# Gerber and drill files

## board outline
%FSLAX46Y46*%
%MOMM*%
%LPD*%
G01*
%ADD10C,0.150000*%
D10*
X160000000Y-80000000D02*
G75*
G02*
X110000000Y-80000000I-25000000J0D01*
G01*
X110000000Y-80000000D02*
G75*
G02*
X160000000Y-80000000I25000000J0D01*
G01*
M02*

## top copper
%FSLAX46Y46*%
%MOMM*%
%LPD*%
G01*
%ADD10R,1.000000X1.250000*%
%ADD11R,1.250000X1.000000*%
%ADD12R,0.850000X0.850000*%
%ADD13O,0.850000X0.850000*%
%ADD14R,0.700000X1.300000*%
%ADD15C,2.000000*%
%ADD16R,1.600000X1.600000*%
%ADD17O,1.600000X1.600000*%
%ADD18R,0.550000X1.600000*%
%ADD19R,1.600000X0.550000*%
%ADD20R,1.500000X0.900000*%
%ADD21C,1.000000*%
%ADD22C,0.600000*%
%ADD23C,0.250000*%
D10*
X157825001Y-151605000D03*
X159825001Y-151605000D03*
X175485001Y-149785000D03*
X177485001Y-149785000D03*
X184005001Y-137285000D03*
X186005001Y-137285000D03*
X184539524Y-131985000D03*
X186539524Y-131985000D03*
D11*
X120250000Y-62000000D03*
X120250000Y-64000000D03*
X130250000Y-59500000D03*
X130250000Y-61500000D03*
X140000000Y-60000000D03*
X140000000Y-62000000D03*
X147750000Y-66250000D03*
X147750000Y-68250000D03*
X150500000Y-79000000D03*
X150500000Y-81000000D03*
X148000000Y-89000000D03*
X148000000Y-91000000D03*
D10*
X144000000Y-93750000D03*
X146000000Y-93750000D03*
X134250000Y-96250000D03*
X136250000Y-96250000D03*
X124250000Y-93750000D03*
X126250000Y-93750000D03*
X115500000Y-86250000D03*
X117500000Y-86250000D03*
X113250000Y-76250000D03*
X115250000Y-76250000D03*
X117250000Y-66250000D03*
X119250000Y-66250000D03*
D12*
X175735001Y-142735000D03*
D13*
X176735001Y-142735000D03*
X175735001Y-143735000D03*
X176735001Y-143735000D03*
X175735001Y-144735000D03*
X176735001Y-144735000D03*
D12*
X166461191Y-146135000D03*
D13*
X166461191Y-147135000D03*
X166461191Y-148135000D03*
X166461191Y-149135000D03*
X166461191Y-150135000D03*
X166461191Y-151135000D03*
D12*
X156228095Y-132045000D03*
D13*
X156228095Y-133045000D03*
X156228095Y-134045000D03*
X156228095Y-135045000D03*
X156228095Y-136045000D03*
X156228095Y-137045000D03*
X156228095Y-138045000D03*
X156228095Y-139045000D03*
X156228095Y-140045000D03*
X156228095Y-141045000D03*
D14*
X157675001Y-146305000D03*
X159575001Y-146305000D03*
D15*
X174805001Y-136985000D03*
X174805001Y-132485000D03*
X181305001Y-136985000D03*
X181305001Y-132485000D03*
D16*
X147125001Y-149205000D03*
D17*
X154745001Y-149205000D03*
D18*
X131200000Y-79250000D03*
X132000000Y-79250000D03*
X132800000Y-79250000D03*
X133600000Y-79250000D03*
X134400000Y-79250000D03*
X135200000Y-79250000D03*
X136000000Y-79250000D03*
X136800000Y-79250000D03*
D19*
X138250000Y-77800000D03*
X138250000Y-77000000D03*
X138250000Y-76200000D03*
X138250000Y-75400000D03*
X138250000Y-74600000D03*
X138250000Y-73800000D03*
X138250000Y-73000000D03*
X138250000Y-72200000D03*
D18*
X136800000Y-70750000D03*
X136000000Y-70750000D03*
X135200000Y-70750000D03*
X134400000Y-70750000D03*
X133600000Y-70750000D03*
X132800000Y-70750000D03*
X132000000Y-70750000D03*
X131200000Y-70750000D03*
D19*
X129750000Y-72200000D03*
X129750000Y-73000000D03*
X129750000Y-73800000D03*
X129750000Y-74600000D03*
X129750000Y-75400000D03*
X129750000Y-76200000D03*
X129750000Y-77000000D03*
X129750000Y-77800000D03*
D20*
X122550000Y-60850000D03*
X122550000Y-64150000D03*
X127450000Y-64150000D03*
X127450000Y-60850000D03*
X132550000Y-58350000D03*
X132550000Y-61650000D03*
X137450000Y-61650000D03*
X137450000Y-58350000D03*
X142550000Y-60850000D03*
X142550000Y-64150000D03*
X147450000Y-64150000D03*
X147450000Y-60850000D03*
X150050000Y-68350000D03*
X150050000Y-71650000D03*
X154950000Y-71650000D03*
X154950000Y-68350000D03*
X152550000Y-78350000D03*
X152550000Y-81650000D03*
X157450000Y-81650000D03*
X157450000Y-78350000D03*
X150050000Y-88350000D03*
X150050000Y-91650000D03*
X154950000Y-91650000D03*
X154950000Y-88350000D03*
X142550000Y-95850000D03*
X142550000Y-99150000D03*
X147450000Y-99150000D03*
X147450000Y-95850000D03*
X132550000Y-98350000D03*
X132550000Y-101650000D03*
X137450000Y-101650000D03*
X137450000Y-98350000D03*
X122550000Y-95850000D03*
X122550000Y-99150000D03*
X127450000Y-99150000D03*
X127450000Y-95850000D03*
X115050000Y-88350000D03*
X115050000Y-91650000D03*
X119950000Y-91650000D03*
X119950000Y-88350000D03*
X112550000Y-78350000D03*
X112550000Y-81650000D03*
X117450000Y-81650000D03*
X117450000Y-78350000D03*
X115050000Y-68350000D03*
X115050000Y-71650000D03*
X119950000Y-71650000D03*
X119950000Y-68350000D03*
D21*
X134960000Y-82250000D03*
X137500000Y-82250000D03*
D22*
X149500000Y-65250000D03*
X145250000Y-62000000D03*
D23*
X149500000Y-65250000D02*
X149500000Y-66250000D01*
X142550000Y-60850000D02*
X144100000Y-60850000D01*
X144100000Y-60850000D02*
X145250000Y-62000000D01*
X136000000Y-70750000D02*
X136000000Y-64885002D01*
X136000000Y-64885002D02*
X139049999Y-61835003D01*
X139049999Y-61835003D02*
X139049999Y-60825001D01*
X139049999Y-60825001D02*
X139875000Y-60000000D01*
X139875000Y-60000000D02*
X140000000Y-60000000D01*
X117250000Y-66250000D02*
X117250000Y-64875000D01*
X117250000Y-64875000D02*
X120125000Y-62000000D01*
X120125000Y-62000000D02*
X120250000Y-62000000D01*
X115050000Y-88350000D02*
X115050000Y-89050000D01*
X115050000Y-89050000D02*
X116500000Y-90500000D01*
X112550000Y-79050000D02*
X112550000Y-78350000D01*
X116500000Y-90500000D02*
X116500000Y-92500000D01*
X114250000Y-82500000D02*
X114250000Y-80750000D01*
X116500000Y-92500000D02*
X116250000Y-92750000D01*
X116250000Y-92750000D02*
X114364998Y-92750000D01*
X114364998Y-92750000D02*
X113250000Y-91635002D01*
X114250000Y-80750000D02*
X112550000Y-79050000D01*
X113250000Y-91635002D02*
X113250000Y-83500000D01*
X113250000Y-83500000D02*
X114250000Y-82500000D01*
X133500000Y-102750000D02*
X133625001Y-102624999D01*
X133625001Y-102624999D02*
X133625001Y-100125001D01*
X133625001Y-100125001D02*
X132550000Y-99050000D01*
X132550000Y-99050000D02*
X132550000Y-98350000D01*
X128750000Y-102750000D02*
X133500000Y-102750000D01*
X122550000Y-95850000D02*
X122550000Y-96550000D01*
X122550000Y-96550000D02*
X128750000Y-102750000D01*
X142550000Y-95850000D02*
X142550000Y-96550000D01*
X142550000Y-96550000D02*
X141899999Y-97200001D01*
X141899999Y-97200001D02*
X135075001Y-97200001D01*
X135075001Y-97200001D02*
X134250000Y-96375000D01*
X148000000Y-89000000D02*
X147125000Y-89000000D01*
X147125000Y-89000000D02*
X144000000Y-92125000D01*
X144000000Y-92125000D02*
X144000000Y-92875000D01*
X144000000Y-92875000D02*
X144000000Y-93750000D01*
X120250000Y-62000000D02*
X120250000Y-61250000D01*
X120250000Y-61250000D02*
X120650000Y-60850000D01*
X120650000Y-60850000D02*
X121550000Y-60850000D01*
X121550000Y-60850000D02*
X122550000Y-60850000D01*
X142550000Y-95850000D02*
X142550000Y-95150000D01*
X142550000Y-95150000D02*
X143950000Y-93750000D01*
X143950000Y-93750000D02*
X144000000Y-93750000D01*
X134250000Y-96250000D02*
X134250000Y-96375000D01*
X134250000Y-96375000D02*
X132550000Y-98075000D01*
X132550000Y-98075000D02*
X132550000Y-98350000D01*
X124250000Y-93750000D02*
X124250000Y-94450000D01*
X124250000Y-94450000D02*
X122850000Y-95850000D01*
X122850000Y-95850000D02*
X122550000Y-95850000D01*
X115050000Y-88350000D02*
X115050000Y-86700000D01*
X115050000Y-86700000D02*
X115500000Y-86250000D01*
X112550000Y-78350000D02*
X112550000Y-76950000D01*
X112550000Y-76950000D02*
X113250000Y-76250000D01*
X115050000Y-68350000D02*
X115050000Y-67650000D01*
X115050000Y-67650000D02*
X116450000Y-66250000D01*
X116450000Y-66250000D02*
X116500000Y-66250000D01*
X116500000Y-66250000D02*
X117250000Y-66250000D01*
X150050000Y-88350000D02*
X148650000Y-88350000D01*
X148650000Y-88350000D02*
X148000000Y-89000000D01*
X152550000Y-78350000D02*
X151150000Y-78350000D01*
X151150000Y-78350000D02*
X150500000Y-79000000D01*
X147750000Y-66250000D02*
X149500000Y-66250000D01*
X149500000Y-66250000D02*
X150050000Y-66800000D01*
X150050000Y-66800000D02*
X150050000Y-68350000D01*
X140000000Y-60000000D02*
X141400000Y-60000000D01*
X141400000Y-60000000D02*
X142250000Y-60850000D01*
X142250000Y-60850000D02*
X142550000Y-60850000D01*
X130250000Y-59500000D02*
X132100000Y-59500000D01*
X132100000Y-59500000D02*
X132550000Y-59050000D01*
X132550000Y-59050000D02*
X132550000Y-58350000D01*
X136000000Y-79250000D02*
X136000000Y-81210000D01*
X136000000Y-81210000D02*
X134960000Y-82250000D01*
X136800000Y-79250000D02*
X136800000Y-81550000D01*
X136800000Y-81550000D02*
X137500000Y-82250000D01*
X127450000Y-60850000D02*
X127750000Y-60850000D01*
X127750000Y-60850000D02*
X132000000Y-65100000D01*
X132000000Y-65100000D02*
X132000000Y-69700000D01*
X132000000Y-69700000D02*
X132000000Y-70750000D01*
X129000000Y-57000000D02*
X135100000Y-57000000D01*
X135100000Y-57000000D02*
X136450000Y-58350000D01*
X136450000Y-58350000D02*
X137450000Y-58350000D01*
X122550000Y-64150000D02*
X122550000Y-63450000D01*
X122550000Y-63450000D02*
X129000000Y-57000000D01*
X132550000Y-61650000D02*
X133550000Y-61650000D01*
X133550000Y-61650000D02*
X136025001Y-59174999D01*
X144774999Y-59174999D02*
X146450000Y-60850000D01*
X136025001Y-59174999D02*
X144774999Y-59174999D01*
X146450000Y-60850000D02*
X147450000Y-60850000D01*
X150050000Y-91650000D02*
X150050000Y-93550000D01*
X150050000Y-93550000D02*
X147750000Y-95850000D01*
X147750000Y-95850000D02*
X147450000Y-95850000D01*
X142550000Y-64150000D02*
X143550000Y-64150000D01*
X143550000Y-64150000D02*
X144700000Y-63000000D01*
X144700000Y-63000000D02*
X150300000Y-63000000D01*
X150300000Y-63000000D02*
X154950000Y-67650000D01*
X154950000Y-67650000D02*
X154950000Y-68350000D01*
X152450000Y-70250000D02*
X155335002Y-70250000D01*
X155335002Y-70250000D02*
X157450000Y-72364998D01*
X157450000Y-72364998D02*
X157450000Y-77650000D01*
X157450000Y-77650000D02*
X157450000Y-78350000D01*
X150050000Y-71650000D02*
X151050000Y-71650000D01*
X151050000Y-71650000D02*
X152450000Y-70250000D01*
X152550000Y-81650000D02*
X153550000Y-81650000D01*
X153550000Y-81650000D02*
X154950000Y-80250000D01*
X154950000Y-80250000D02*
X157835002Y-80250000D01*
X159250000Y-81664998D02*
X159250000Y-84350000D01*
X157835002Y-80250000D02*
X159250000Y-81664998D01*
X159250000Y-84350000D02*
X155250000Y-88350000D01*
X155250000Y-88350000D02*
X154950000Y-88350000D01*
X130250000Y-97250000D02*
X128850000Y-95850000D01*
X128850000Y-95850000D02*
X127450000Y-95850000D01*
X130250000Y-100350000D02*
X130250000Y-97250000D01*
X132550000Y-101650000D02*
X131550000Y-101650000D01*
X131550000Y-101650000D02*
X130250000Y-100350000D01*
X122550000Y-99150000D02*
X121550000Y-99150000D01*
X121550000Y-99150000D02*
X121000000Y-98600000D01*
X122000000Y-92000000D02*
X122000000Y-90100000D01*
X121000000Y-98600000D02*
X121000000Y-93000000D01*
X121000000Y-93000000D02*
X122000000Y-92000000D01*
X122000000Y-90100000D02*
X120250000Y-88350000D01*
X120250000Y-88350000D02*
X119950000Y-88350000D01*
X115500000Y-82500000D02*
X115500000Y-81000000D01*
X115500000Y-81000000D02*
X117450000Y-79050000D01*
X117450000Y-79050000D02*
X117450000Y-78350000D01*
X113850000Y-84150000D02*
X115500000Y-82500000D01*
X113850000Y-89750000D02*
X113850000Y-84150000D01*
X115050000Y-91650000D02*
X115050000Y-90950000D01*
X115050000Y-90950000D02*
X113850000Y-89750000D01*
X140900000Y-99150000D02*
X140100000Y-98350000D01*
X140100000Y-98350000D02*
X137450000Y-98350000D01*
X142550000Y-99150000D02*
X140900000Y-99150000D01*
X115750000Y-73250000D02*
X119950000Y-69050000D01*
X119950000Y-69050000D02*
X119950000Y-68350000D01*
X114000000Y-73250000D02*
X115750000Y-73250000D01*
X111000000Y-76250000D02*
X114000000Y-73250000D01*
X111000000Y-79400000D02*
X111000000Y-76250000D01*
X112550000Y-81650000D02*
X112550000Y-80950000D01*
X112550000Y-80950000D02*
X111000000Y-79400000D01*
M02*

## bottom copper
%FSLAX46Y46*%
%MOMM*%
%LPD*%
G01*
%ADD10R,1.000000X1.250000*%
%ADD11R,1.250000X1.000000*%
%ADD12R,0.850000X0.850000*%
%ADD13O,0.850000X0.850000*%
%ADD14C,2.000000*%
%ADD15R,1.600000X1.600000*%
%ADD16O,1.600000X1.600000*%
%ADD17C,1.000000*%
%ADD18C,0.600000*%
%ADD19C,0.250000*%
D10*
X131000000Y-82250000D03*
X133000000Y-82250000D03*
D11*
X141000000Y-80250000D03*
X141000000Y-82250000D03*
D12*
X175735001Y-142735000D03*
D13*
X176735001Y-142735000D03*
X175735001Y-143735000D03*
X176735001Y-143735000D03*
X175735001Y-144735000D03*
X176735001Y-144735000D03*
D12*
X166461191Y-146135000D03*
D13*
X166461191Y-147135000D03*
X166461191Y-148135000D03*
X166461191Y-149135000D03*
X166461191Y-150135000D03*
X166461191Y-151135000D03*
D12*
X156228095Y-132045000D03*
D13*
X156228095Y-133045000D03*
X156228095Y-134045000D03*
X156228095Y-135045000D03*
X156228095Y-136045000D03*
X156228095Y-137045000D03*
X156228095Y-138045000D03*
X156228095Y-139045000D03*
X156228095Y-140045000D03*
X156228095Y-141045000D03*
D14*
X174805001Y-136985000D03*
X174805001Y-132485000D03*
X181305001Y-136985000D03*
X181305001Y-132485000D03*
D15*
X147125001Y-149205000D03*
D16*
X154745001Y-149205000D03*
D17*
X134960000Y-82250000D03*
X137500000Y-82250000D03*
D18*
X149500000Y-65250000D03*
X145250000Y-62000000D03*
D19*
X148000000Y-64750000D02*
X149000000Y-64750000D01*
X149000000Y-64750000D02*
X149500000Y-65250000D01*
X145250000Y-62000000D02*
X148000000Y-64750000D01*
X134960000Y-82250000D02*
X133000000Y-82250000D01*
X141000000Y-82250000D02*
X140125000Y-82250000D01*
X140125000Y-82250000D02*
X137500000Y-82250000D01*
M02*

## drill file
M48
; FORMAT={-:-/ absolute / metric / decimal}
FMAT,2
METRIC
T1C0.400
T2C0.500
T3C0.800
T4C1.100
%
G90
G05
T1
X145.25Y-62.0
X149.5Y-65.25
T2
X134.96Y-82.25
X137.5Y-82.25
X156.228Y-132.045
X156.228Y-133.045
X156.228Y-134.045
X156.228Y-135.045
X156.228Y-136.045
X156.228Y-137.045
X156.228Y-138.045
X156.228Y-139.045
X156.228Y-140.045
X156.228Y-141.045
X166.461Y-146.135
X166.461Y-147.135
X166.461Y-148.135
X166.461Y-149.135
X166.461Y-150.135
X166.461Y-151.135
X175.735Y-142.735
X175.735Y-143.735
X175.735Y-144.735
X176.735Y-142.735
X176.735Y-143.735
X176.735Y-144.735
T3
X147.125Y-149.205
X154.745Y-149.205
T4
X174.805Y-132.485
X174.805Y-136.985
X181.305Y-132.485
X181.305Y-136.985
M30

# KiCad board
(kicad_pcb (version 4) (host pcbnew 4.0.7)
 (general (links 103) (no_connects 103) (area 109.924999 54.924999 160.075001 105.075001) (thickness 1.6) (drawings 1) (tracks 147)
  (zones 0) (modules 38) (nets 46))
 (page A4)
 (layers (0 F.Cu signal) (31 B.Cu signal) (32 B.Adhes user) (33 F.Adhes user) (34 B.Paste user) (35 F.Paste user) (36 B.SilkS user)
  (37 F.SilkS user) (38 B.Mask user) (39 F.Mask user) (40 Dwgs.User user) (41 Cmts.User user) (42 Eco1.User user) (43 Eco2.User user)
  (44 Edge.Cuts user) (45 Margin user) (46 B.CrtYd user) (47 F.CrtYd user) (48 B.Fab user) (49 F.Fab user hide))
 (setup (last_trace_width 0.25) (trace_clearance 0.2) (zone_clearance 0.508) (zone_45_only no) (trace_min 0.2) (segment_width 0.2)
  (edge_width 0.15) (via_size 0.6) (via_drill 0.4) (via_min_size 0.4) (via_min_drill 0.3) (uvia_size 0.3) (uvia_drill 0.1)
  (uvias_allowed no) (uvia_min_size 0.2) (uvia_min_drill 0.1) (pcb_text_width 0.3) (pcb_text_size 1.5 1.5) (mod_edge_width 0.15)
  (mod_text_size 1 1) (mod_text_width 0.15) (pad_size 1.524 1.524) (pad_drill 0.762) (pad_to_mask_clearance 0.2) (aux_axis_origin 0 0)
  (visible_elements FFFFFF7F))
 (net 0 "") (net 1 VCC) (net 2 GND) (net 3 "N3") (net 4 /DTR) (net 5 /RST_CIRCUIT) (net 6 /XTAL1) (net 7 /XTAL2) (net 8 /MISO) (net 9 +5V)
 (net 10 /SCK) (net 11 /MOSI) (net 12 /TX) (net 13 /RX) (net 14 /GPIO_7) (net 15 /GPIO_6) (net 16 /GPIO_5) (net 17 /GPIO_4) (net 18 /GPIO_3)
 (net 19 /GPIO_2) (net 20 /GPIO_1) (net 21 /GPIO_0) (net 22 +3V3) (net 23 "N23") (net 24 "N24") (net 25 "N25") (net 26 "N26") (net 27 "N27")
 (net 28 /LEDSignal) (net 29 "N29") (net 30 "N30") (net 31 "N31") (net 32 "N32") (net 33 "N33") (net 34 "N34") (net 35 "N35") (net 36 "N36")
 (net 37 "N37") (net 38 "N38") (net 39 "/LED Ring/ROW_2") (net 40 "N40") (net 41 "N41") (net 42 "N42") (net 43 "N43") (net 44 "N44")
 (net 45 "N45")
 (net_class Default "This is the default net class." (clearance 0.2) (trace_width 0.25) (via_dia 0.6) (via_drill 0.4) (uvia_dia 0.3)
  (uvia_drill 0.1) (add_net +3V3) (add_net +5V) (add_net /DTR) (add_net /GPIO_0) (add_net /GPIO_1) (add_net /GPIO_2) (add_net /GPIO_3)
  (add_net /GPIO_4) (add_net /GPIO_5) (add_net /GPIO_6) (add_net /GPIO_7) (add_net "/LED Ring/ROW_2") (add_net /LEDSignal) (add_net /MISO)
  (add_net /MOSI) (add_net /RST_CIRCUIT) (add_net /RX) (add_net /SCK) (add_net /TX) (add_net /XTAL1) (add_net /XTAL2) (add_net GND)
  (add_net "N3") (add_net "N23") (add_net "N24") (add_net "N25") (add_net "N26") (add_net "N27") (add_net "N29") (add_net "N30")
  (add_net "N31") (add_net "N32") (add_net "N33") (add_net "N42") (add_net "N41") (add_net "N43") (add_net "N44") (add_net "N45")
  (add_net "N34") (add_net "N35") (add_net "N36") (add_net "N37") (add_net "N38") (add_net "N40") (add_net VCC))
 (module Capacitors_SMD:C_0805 (layer F.Cu) (at 158.825001 151.605)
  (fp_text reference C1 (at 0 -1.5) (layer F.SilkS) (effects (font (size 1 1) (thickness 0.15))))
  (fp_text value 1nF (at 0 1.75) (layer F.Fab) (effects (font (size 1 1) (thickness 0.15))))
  (pad 1 smd rect (at -1 0) (size 1 1.25) (layers F.Cu F.Paste F.Mask) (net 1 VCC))
  (pad 2 smd rect (at 1 0) (size 1 1.25) (layers F.Cu F.Paste F.Mask) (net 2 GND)))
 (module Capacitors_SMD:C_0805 (layer F.Cu) (at 176.485001 149.785)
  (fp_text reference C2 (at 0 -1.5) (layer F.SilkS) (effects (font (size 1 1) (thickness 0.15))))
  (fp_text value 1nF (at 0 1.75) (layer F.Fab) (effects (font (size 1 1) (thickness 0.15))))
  (pad 1 smd rect (at -1 0) (size 1 1.25) (layers F.Cu F.Paste F.Mask) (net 1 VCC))
  (pad 2 smd rect (at 1 0) (size 1 1.25) (layers F.Cu F.Paste F.Mask) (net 2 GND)))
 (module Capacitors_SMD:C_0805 (layer F.Cu) (at 185.005001 137.285)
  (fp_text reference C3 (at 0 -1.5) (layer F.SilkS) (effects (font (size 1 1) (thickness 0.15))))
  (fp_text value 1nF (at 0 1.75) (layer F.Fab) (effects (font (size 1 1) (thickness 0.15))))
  (pad 1 smd rect (at -1 0) (size 1 1.25) (layers F.Cu F.Paste F.Mask) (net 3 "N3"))
  (pad 2 smd rect (at 1 0) (size 1 1.25) (layers F.Cu F.Paste F.Mask) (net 2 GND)))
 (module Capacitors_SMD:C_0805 (layer F.Cu) (at 185.539524 131.985)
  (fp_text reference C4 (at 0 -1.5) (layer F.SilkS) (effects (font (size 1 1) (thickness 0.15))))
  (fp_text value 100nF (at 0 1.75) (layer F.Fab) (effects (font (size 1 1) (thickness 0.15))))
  (pad 1 smd rect (at -1 0) (size 1 1.25) (layers F.Cu F.Paste F.Mask) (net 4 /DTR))
  (pad 2 smd rect (at 1 0) (size 1 1.25) (layers F.Cu F.Paste F.Mask) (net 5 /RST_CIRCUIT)))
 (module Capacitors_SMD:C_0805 (layer B.Cu) (at 132 82.25)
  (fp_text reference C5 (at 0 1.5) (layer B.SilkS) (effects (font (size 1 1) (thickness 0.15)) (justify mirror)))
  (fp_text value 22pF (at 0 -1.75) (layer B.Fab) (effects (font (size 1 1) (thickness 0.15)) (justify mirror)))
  (pad 1 smd rect (at -1 0) (size 1 1.25) (layers B.Cu B.Paste B.Mask) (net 2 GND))
  (pad 2 smd rect (at 1 0) (size 1 1.25) (layers B.Cu B.Paste B.Mask) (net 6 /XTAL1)))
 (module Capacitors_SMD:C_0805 (layer B.Cu) (at 141 81.25 270)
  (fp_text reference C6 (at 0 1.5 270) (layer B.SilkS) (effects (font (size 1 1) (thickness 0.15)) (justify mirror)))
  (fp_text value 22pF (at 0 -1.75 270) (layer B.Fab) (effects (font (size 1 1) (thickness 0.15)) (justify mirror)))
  (pad 1 smd rect (at -1 0 270) (size 1 1.25) (layers B.Cu B.Paste B.Mask) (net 2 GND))
  (pad 2 smd rect (at 1 0 270) (size 1 1.25) (layers B.Cu B.Paste B.Mask) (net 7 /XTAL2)))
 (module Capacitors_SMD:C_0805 (layer F.Cu) (at 120.25 63 270)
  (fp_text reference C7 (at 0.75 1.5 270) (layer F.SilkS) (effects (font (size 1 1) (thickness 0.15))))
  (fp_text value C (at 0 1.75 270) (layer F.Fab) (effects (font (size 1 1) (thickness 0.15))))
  (pad 1 smd rect (at -1 0 270) (size 1 1.25) (layers F.Cu F.Paste F.Mask) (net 1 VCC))
  (pad 2 smd rect (at 1 0 270) (size 1 1.25) (layers F.Cu F.Paste F.Mask) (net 2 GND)))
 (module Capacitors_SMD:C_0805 (layer F.Cu) (at 130.25 60.5 270)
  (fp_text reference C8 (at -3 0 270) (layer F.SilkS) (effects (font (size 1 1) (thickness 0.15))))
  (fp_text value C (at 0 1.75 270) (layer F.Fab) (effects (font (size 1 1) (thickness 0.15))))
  (pad 1 smd rect (at -1 0 270) (size 1 1.25) (layers F.Cu F.Paste F.Mask) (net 1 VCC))
  (pad 2 smd rect (at 1 0 270) (size 1 1.25) (layers F.Cu F.Paste F.Mask) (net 2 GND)))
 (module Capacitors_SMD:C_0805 (layer F.Cu) (at 140 61 270)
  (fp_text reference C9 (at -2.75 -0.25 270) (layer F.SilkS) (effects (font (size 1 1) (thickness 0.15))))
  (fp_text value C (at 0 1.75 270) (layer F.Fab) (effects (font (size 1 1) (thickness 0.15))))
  (pad 1 smd rect (at -1 0 270) (size 1 1.25) (layers F.Cu F.Paste F.Mask) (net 1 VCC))
  (pad 2 smd rect (at 1 0 270) (size 1 1.25) (layers F.Cu F.Paste F.Mask) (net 2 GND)))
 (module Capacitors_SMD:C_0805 (layer F.Cu) (at 147.75 67.25 270)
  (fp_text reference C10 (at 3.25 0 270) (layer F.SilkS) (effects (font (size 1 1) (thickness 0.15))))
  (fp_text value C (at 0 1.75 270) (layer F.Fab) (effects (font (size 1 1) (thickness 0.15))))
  (pad 1 smd rect (at -1 0 270) (size 1 1.25) (layers F.Cu F.Paste F.Mask) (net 1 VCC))
  (pad 2 smd rect (at 1 0 270) (size 1 1.25) (layers F.Cu F.Paste F.Mask) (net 2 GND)))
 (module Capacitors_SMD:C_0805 (layer F.Cu) (at 150.5 80 270)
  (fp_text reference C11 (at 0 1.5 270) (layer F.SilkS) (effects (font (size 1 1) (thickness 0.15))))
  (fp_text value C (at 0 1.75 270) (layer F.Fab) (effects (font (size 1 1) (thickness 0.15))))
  (pad 1 smd rect (at -1 0 270) (size 1 1.25) (layers F.Cu F.Paste F.Mask) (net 1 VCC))
  (pad 2 smd rect (at 1 0 270) (size 1 1.25) (layers F.Cu F.Paste F.Mask) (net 2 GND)))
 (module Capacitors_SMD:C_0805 (layer F.Cu) (at 148 90 270)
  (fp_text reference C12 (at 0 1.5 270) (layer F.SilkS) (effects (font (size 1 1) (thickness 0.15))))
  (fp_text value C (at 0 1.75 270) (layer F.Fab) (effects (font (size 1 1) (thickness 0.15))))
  (pad 1 smd rect (at -1 0 270) (size 1 1.25) (layers F.Cu F.Paste F.Mask) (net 1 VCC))
  (pad 2 smd rect (at 1 0 270) (size 1 1.25) (layers F.Cu F.Paste F.Mask) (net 2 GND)))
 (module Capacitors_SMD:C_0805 (layer F.Cu) (at 145 93.75)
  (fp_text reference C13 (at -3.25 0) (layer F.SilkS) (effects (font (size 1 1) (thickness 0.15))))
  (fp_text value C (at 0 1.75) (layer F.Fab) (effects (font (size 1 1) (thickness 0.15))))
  (pad 1 smd rect (at -1 0) (size 1 1.25) (layers F.Cu F.Paste F.Mask) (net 1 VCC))
  (pad 2 smd rect (at 1 0) (size 1 1.25) (layers F.Cu F.Paste F.Mask) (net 2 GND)))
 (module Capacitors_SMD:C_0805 (layer F.Cu) (at 135.25 96.25)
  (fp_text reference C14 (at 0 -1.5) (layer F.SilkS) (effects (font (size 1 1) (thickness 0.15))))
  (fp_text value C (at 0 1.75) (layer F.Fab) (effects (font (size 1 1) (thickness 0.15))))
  (pad 1 smd rect (at -1 0) (size 1 1.25) (layers F.Cu F.Paste F.Mask) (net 1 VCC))
  (pad 2 smd rect (at 1 0) (size 1 1.25) (layers F.Cu F.Paste F.Mask) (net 2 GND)))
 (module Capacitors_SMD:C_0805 (layer F.Cu) (at 125.25 93.75)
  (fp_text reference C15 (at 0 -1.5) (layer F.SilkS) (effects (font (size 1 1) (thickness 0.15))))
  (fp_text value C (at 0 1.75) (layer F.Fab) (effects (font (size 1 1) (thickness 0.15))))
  (pad 1 smd rect (at -1 0) (size 1 1.25) (layers F.Cu F.Paste F.Mask) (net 1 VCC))
  (pad 2 smd rect (at 1 0) (size 1 1.25) (layers F.Cu F.Paste F.Mask) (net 2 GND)))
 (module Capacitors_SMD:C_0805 (layer F.Cu) (at 116.5 86.25)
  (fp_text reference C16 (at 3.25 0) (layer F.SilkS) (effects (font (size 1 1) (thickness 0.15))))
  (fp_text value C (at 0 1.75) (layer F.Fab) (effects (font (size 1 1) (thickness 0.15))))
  (pad 1 smd rect (at -1 0) (size 1 1.25) (layers F.Cu F.Paste F.Mask) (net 1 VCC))
  (pad 2 smd rect (at 1 0) (size 1 1.25) (layers F.Cu F.Paste F.Mask) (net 2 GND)))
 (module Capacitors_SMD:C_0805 (layer F.Cu) (at 114.25 76.25)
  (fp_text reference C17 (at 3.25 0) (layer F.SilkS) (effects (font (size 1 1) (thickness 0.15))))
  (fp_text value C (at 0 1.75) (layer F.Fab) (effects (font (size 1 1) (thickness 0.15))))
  (pad 1 smd rect (at -1 0) (size 1 1.25) (layers F.Cu F.Paste F.Mask) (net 1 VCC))
  (pad 2 smd rect (at 1 0) (size 1 1.25) (layers F.Cu F.Paste F.Mask) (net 2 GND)))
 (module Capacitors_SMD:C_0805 (layer F.Cu) (at 118.25 66.25)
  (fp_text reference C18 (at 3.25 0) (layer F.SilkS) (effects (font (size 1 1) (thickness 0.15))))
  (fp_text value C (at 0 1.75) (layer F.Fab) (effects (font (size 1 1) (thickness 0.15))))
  (pad 1 smd rect (at -1 0) (size 1 1.25) (layers F.Cu F.Paste F.Mask) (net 1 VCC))
  (pad 2 smd rect (at 1 0) (size 1 1.25) (layers F.Cu F.Paste F.Mask) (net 2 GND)))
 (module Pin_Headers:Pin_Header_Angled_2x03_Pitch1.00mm (layer F.Cu) (at 175.735001 142.735)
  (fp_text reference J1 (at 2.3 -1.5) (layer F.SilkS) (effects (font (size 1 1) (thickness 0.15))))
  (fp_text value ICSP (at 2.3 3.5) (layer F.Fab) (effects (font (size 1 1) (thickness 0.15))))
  (pad 1 thru_hole rect (at 0 0) (size 0.85 0.85) (drill 0.5) (layers *.Cu *.Mask) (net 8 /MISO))
  (pad 2 thru_hole oval (at 1 0) (size 0.85 0.85) (drill 0.5) (layers *.Cu *.Mask) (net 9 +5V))
  (pad 3 thru_hole oval (at 0 1) (size 0.85 0.85) (drill 0.5) (layers *.Cu *.Mask) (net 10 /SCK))
  (pad 4 thru_hole oval (at 1 1) (size 0.85 0.85) (drill 0.5) (layers *.Cu *.Mask) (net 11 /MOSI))
  (pad 5 thru_hole oval (at 0 2) (size 0.85 0.85) (drill 0.5) (layers *.Cu *.Mask) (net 5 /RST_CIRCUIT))
  (pad 6 thru_hole oval (at 1 2) (size 0.85 0.85) (drill 0.5) (layers *.Cu *.Mask) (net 2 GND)))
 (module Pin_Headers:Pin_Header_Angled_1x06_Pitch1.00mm (layer F.Cu) (at 166.461191 146.135)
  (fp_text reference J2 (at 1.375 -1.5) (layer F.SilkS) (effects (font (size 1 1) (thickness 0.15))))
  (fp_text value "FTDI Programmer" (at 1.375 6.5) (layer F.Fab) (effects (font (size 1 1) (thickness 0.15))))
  (pad 1 thru_hole rect (at 0 0) (size 0.85 0.85) (drill 0.5) (layers *.Cu *.Mask) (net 4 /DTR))
  (pad 2 thru_hole oval (at 0 1) (size 0.85 0.85) (drill 0.5) (layers *.Cu *.Mask) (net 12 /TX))
  (pad 3 thru_hole oval (at 0 2) (size 0.85 0.85) (drill 0.5) (layers *.Cu *.Mask) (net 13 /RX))
  (pad 4 thru_hole oval (at 0 3) (size 0.85 0.85) (drill 0.5) (layers *.Cu *.Mask) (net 9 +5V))
  (pad 5 thru_hole oval (at 0 4) (size 0.85 0.85) (drill 0.5) (layers *.Cu *.Mask) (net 2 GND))
  (pad 6 thru_hole oval (at 0 5) (size 0.85 0.85) (drill 0.5) (layers *.Cu *.Mask) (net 2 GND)))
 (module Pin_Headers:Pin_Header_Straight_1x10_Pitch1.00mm (layer F.Cu) (at 156.228095 132.045)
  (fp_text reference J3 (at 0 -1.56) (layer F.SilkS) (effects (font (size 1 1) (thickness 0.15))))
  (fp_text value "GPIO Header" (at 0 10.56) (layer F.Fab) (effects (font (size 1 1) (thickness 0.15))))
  (pad 1 thru_hole rect (at 0 0) (size 0.85 0.85) (drill 0.5) (layers *.Cu *.Mask) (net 2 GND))
  (pad 2 thru_hole oval (at 0 1) (size 0.85 0.85) (drill 0.5) (layers *.Cu *.Mask) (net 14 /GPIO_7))
  (pad 3 thru_hole oval (at 0 2) (size 0.85 0.85) (drill 0.5) (layers *.Cu *.Mask) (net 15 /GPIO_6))
  (pad 4 thru_hole oval (at 0 3) (size 0.85 0.85) (drill 0.5) (layers *.Cu *.Mask) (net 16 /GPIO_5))
  (pad 5 thru_hole oval (at 0 4) (size 0.85 0.85) (drill 0.5) (layers *.Cu *.Mask) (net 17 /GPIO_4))
  (pad 6 thru_hole oval (at 0 5) (size 0.85 0.85) (drill 0.5) (layers *.Cu *.Mask) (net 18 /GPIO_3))
  (pad 7 thru_hole oval (at 0 6) (size 0.85 0.85) (drill 0.5) (layers *.Cu *.Mask) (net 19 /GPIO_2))
  (pad 8 thru_hole oval (at 0 7) (size 0.85 0.85) (drill 0.5) (layers *.Cu *.Mask) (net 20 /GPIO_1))
  (pad 9 thru_hole oval (at 0 8) (size 0.85 0.85) (drill 0.5) (layers *.Cu *.Mask) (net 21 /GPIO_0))
  (pad 10 thru_hole oval (at 0 9) (size 0.85 0.85) (drill 0.5) (layers *.Cu *.Mask) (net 1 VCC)))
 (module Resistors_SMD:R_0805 (layer F.Cu) (at 158.625001 146.305)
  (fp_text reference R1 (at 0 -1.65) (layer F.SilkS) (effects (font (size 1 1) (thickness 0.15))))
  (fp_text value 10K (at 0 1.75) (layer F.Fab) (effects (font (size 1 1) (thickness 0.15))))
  (pad 1 smd rect (at -0.95 0) (size 0.7 1.3) (layers F.Cu F.Paste F.Mask) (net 9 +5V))
  (pad 2 smd rect (at 0.95 0) (size 0.7 1.3) (layers F.Cu F.Paste F.Mask) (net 5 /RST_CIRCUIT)))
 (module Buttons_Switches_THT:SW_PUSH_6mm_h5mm (layer F.Cu) (at 174.805001 132.485)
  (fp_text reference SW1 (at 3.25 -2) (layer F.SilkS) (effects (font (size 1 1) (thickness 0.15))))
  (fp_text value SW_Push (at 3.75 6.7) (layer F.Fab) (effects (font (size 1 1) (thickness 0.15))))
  (pad 2 thru_hole circle (at 0 4.5 90) (size 2 2) (drill 1.1) (layers *.Cu *.Mask) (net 2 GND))
  (pad 1 thru_hole circle (at 0 0 90) (size 2 2) (drill 1.1) (layers *.Cu *.Mask) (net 5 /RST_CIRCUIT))
  (pad 2 thru_hole circle (at 6.5 4.5 90) (size 2 2) (drill 1.1) (layers *.Cu *.Mask) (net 2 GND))
  (pad 1 thru_hole circle (at 6.5 0 90) (size 2 2) (drill 1.1) (layers *.Cu *.Mask) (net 5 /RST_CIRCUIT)))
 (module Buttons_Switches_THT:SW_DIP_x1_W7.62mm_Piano (layer F.Cu) (at 147.125001 149.205)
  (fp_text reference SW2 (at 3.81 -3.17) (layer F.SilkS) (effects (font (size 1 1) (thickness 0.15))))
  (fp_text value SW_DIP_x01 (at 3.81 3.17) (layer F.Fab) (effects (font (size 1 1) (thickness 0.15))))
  (pad 1 thru_hole rect (at 0 0) (size 1.6 1.6) (drill 0.8) (layers *.Cu *.Mask) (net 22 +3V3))
  (pad 2 thru_hole oval (at 7.62 0) (size 1.6 1.6) (drill 0.8) (layers *.Cu *.Mask) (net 1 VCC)))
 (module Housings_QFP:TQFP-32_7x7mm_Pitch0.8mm (layer F.Cu) (at 134 75 90)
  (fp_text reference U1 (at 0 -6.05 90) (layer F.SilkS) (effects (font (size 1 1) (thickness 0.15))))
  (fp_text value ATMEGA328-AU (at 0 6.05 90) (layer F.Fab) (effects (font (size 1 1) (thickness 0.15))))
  (pad 1 smd rect (at -4.25 -2.8 90) (size 1.6 0.55) (layers F.Cu F.Paste F.Mask) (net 18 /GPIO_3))
  (pad 2 smd rect (at -4.25 -2 90) (size 1.6 0.55) (layers F.Cu F.Paste F.Mask) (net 17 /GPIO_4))
  (pad 3 smd rect (at -4.25 -1.2 90) (size 1.6 0.55) (layers F.Cu F.Paste F.Mask) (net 2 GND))
  (pad 4 smd rect (at -4.25 -0.4 90) (size 1.6 0.55) (layers F.Cu F.Paste F.Mask) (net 1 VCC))
  (pad 5 smd rect (at -4.25 0.4 90) (size 1.6 0.55) (layers F.Cu F.Paste F.Mask) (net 2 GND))
  (pad 6 smd rect (at -4.25 1.2 90) (size 1.6 0.55) (layers F.Cu F.Paste F.Mask) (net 1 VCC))
  (pad 7 smd rect (at -4.25 2 90) (size 1.6 0.55) (layers F.Cu F.Paste F.Mask) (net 6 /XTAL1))
  (pad 8 smd rect (at -4.25 2.8 90) (size 1.6 0.55) (layers F.Cu F.Paste F.Mask) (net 7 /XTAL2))
  (pad 9 smd rect (at -2.8 4.25 180) (size 1.6 0.55) (layers F.Cu F.Paste F.Mask) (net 16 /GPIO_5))
  (pad 10 smd rect (at -2 4.25 180) (size 1.6 0.55) (layers F.Cu F.Paste F.Mask) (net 15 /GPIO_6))
  (pad 11 smd rect (at -1.2 4.25 180) (size 1.6 0.55) (layers F.Cu F.Paste F.Mask) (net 14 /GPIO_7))
  (pad 12 smd rect (at -0.4 4.25 180) (size 1.6 0.55) (layers F.Cu F.Paste F.Mask) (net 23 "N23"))
  (pad 13 smd rect (at 0.4 4.25 180) (size 1.6 0.55) (layers F.Cu F.Paste F.Mask) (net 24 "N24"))
  (pad 14 smd rect (at 1.2 4.25 180) (size 1.6 0.55) (layers F.Cu F.Paste F.Mask) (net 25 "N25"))
  (pad 15 smd rect (at 2 4.25 180) (size 1.6 0.55) (layers F.Cu F.Paste F.Mask) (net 11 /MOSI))
  (pad 16 smd rect (at 2.8 4.25 180) (size 1.6 0.55) (layers F.Cu F.Paste F.Mask) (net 8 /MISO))
  (pad 17 smd rect (at 4.25 2.8 90) (size 1.6 0.55) (layers F.Cu F.Paste F.Mask) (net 10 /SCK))
  (pad 18 smd rect (at 4.25 2 90) (size 1.6 0.55) (layers F.Cu F.Paste F.Mask) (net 1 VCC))
  (pad 19 smd rect (at 4.25 1.2 90) (size 1.6 0.55) (layers F.Cu F.Paste F.Mask) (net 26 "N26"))
  (pad 20 smd rect (at 4.25 0.4 90) (size 1.6 0.55) (layers F.Cu F.Paste F.Mask) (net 3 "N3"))
  (pad 21 smd rect (at 4.25 -0.4 90) (size 1.6 0.55) (layers F.Cu F.Paste F.Mask) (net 2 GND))
  (pad 22 smd rect (at 4.25 -1.2 90) (size 1.6 0.55) (layers F.Cu F.Paste F.Mask) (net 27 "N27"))
  (pad 23 smd rect (at 4.25 -2 90) (size 1.6 0.55) (layers F.Cu F.Paste F.Mask) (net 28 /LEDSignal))
  (pad 24 smd rect (at 4.25 -2.8 90) (size 1.6 0.55) (layers F.Cu F.Paste F.Mask) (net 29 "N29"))
  (pad 25 smd rect (at 2.8 -4.25 180) (size 1.6 0.55) (layers F.Cu F.Paste F.Mask) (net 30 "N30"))
  (pad 26 smd rect (at 2 -4.25 180) (size 1.6 0.55) (layers F.Cu F.Paste F.Mask) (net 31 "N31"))
  (pad 27 smd rect (at 1.2 -4.25 180) (size 1.6 0.55) (layers F.Cu F.Paste F.Mask) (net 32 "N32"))
  (pad 28 smd rect (at 0.4 -4.25 180) (size 1.6 0.55) (layers F.Cu F.Paste F.Mask) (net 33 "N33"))
  (pad 29 smd rect (at -0.4 -4.25 180) (size 1.6 0.55) (layers F.Cu F.Paste F.Mask) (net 5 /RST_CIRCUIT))
  (pad 30 smd rect (at -1.2 -4.25 180) (size 1.6 0.55) (layers F.Cu F.Paste F.Mask) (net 21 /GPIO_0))
  (pad 31 smd rect (at -2 -4.25 180) (size 1.6 0.55) (layers F.Cu F.Paste F.Mask) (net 20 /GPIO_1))
  (pad 32 smd rect (at -2.8 -4.25 180) (size 1.6 0.55) (layers F.Cu F.Paste F.Mask) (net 19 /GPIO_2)))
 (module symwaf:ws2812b (layer F.Cu) (at 125 62.5)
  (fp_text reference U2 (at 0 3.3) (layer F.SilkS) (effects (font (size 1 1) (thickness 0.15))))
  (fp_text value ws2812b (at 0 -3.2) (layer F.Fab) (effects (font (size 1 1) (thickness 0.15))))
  (pad 1 smd rect (at -2.45 -1.65) (size 1.5 0.9) (layers F.Cu F.Paste F.Mask) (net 1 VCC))
  (pad 2 smd rect (at -2.45 1.65) (size 1.5 0.9) (layers F.Cu F.Paste F.Mask) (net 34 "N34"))
  (pad 3 smd rect (at 2.45 1.65) (size 1.5 0.9) (layers F.Cu F.Paste F.Mask) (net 2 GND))
  (pad 4 smd rect (at 2.45 -1.65) (size 1.5 0.9) (layers F.Cu F.Paste F.Mask) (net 28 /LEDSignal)))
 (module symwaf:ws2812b (layer F.Cu) (at 135 60)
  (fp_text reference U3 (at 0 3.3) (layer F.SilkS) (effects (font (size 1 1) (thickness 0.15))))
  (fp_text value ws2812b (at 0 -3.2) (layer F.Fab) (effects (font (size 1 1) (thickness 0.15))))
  (pad 1 smd rect (at -2.45 -1.65) (size 1.5 0.9) (layers F.Cu F.Paste F.Mask) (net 1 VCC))
  (pad 2 smd rect (at -2.45 1.65) (size 1.5 0.9) (layers F.Cu F.Paste F.Mask) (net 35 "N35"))
  (pad 3 smd rect (at 2.45 1.65) (size 1.5 0.9) (layers F.Cu F.Paste F.Mask) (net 2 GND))
  (pad 4 smd rect (at 2.45 -1.65) (size 1.5 0.9) (layers F.Cu F.Paste F.Mask) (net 34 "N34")))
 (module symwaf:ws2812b (layer F.Cu) (at 145 62.5)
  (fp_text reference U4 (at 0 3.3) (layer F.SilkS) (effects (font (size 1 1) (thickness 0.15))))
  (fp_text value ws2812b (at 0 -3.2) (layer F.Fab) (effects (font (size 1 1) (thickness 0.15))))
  (pad 1 smd rect (at -2.45 -1.65) (size 1.5 0.9) (layers F.Cu F.Paste F.Mask) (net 1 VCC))
  (pad 2 smd rect (at -2.45 1.65) (size 1.5 0.9) (layers F.Cu F.Paste F.Mask) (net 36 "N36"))
  (pad 3 smd rect (at 2.45 1.65) (size 1.5 0.9) (layers F.Cu F.Paste F.Mask) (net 2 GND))
  (pad 4 smd rect (at 2.45 -1.65) (size 1.5 0.9) (layers F.Cu F.Paste F.Mask) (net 35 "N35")))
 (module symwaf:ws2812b (layer F.Cu) (at 152.5 70)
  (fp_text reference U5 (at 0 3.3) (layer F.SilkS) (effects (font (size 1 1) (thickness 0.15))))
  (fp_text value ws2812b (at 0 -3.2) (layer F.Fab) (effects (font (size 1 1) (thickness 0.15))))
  (pad 1 smd rect (at -2.45 -1.65) (size 1.5 0.9) (layers F.Cu F.Paste F.Mask) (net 1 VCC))
  (pad 2 smd rect (at -2.45 1.65) (size 1.5 0.9) (layers F.Cu F.Paste F.Mask) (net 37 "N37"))
  (pad 3 smd rect (at 2.45 1.65) (size 1.5 0.9) (layers F.Cu F.Paste F.Mask) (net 2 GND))
  (pad 4 smd rect (at 2.45 -1.65) (size 1.5 0.9) (layers F.Cu F.Paste F.Mask) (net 36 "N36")))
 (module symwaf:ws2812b (layer F.Cu) (at 155 80)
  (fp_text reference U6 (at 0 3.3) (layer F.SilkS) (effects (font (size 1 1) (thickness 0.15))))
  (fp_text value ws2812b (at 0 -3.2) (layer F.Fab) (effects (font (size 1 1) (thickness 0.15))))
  (pad 1 smd rect (at -2.45 -1.65) (size 1.5 0.9) (layers F.Cu F.Paste F.Mask) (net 1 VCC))
  (pad 2 smd rect (at -2.45 1.65) (size 1.5 0.9) (layers F.Cu F.Paste F.Mask) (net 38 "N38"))
  (pad 3 smd rect (at 2.45 1.65) (size 1.5 0.9) (layers F.Cu F.Paste F.Mask) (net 2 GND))
  (pad 4 smd rect (at 2.45 -1.65) (size 1.5 0.9) (layers F.Cu F.Paste F.Mask) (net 37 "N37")))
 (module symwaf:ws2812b (layer F.Cu) (at 152.5 90)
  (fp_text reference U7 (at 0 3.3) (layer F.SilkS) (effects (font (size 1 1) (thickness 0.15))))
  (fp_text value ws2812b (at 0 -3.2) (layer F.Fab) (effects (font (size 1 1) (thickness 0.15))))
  (pad 1 smd rect (at -2.45 -1.65) (size 1.5 0.9) (layers F.Cu F.Paste F.Mask) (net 1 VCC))
  (pad 2 smd rect (at -2.45 1.65) (size 1.5 0.9) (layers F.Cu F.Paste F.Mask) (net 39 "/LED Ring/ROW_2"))
  (pad 3 smd rect (at 2.45 1.65) (size 1.5 0.9) (layers F.Cu F.Paste F.Mask) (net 2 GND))
  (pad 4 smd rect (at 2.45 -1.65) (size 1.5 0.9) (layers F.Cu F.Paste F.Mask) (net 38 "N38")))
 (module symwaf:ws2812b (layer F.Cu) (at 145 97.5)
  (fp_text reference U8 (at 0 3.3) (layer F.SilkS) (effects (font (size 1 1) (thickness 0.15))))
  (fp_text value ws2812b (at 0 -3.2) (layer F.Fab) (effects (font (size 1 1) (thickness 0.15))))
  (pad 1 smd rect (at -2.45 -1.65) (size 1.5 0.9) (layers F.Cu F.Paste F.Mask) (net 1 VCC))
  (pad 2 smd rect (at -2.45 1.65) (size 1.5 0.9) (layers F.Cu F.Paste F.Mask) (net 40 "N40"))
  (pad 3 smd rect (at 2.45 1.65) (size 1.5 0.9) (layers F.Cu F.Paste F.Mask) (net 2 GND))
  (pad 4 smd rect (at 2.45 -1.65) (size 1.5 0.9) (layers F.Cu F.Paste F.Mask) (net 39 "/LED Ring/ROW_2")))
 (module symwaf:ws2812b (layer F.Cu) (at 135 100)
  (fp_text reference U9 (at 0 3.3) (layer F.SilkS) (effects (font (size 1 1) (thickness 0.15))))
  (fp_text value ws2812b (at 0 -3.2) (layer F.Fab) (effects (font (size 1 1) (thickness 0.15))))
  (pad 1 smd rect (at -2.45 -1.65) (size 1.5 0.9) (layers F.Cu F.Paste F.Mask) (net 1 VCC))
  (pad 2 smd rect (at -2.45 1.65) (size 1.5 0.9) (layers F.Cu F.Paste F.Mask) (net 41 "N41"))
  (pad 3 smd rect (at 2.45 1.65) (size 1.5 0.9) (layers F.Cu F.Paste F.Mask) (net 2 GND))
  (pad 4 smd rect (at 2.45 -1.65) (size 1.5 0.9) (layers F.Cu F.Paste F.Mask) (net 40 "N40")))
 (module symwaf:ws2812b (layer F.Cu) (at 125 97.5)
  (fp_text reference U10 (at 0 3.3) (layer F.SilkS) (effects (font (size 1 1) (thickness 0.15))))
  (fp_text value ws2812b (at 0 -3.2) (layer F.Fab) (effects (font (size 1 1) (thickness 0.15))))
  (pad 1 smd rect (at -2.45 -1.65) (size 1.5 0.9) (layers F.Cu F.Paste F.Mask) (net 1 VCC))
  (pad 2 smd rect (at -2.45 1.65) (size 1.5 0.9) (layers F.Cu F.Paste F.Mask) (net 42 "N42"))
  (pad 3 smd rect (at 2.45 1.65) (size 1.5 0.9) (layers F.Cu F.Paste F.Mask) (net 2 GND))
  (pad 4 smd rect (at 2.45 -1.65) (size 1.5 0.9) (layers F.Cu F.Paste F.Mask) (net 41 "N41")))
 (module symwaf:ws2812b (layer F.Cu) (at 117.5 90)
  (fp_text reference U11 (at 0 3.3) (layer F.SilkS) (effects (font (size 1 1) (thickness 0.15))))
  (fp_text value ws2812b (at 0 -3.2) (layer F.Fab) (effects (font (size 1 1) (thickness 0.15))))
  (pad 1 smd rect (at -2.45 -1.65) (size 1.5 0.9) (layers F.Cu F.Paste F.Mask) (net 1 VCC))
  (pad 2 smd rect (at -2.45 1.65) (size 1.5 0.9) (layers F.Cu F.Paste F.Mask) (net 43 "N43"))
  (pad 3 smd rect (at 2.45 1.65) (size 1.5 0.9) (layers F.Cu F.Paste F.Mask) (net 2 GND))
  (pad 4 smd rect (at 2.45 -1.65) (size 1.5 0.9) (layers F.Cu F.Paste F.Mask) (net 42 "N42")))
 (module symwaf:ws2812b (layer F.Cu) (at 115 80)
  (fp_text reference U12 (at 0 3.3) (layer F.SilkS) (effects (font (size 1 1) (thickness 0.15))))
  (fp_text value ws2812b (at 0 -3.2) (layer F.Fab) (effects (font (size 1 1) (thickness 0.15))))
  (pad 1 smd rect (at -2.45 -1.65) (size 1.5 0.9) (layers F.Cu F.Paste F.Mask) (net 1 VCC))
  (pad 2 smd rect (at -2.45 1.65) (size 1.5 0.9) (layers F.Cu F.Paste F.Mask) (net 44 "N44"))
  (pad 3 smd rect (at 2.45 1.65) (size 1.5 0.9) (layers F.Cu F.Paste F.Mask) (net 2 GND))
  (pad 4 smd rect (at 2.45 -1.65) (size 1.5 0.9) (layers F.Cu F.Paste F.Mask) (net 43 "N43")))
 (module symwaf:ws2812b (layer F.Cu) (at 117.5 70)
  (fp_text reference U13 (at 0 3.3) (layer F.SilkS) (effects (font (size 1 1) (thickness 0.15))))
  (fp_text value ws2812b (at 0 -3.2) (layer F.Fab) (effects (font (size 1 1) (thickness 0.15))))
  (pad 1 smd rect (at -2.45 -1.65) (size 1.5 0.9) (layers F.Cu F.Paste F.Mask) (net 1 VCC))
  (pad 2 smd rect (at -2.45 1.65) (size 1.5 0.9) (layers F.Cu F.Paste F.Mask) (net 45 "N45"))
  (pad 3 smd rect (at 2.45 1.65) (size 1.5 0.9) (layers F.Cu F.Paste F.Mask) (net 2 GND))
  (pad 4 smd rect (at 2.45 -1.65) (size 1.5 0.9) (layers F.Cu F.Paste F.Mask) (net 44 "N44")))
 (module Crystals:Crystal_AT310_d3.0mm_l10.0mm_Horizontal (layer B.Cu) (at 134.96 82.25)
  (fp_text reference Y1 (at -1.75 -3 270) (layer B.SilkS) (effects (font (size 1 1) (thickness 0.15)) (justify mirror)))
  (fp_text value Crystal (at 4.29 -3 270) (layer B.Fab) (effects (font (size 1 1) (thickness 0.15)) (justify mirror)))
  (pad 1 thru_hole circle (at 0 0) (size 1 1) (drill 0.5) (layers *.Cu *.Mask) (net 6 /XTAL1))
  (pad 2 thru_hole circle (at 2.54 0) (size 1 1) (drill 0.5) (layers *.Cu *.Mask) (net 7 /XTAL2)))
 (gr_circle (center 135 80) (end 160 80) (layer Edge.Cuts) (width 0.15))
 (segment (start 149.5 65.25) (end 149.5 66.25) (width 0.25) (layer F.Cu) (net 1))
 (segment (start 148 64.75) (end 149 64.75) (width 0.25) (layer B.Cu) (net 1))
 (segment (start 149 64.75) (end 149.5 65.25) (width 0.25) (layer B.Cu) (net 1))
 (via (at 149.5 65.25) (size 0.6) (drill 0.4) (layers F.Cu B.Cu) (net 1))
 (segment (start 145.25 62) (end 148 64.75) (width 0.25) (layer B.Cu) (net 1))
 (segment (start 142.55 60.85) (end 144.1 60.85) (width 0.25) (layer F.Cu) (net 1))
 (segment (start 144.1 60.85) (end 145.25 62) (width 0.25) (layer F.Cu) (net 1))
 (via (at 145.25 62) (size 0.6) (drill 0.4) (layers F.Cu B.Cu) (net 1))
 (segment (start 136 70.75) (end 136 64.885002) (width 0.25) (layer F.Cu) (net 1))
 (segment (start 136 64.885002) (end 139.049999 61.835003) (width 0.25) (layer F.Cu) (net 1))
 (segment (start 139.049999 61.835003) (end 139.049999 60.825001) (width 0.25) (layer F.Cu) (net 1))
 (segment (start 139.049999 60.825001) (end 139.875 60) (width 0.25) (layer F.Cu) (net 1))
 (segment (start 139.875 60) (end 140 60) (width 0.25) (layer F.Cu) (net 1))
 (segment (start 117.25 66.25) (end 117.25 64.875) (width 0.25) (layer F.Cu) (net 1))
 (segment (start 117.25 64.875) (end 120.125 62) (width 0.25) (layer F.Cu) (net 1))
 (segment (start 120.125 62) (end 120.25 62) (width 0.25) (layer F.Cu) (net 1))
 (segment (start 115.05 88.35) (end 115.05 89.05) (width 0.25) (layer F.Cu) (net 1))
 (segment (start 115.05 89.05) (end 116.5 90.5) (width 0.25) (layer F.Cu) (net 1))
 (segment (start 112.55 79.05) (end 112.55 78.35) (width 0.25) (layer F.Cu) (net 1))
 (segment (start 116.5 90.5) (end 116.5 92.5) (width 0.25) (layer F.Cu) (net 1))
 (segment (start 114.25 82.5) (end 114.25 80.75) (width 0.25) (layer F.Cu) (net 1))
 (segment (start 116.5 92.5) (end 116.25 92.75) (width 0.25) (layer F.Cu) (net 1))
 (segment (start 116.25 92.75) (end 114.364998 92.75) (width 0.25) (layer F.Cu) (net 1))
 (segment (start 114.364998 92.75) (end 113.25 91.635002) (width 0.25) (layer F.Cu) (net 1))
 (segment (start 114.25 80.75) (end 112.55 79.05) (width 0.25) (layer F.Cu) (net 1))
 (segment (start 113.25 91.635002) (end 113.25 83.5) (width 0.25) (layer F.Cu) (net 1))
 (segment (start 113.25 83.5) (end 114.25 82.5) (width 0.25) (layer F.Cu) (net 1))
 (segment (start 133.5 102.75) (end 133.625001 102.624999) (width 0.25) (layer F.Cu) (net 1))
 (segment (start 133.625001 102.624999) (end 133.625001 100.125001) (width 0.25) (layer F.Cu) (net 1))
 (segment (start 133.625001 100.125001) (end 132.55 99.05) (width 0.25) (layer F.Cu) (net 1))
 (segment (start 132.55 99.05) (end 132.55 98.35) (width 0.25) (layer F.Cu) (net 1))
 (segment (start 128.75 102.75) (end 133.5 102.75) (width 0.25) (layer F.Cu) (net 1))
 (segment (start 122.55 95.85) (end 122.55 96.55) (width 0.25) (layer F.Cu) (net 1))
 (segment (start 122.55 96.55) (end 128.75 102.75) (width 0.25) (layer F.Cu) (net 1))
 (segment (start 142.55 95.85) (end 142.55 96.55) (width 0.25) (layer F.Cu) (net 1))
 (segment (start 142.55 96.55) (end 141.899999 97.200001) (width 0.25) (layer F.Cu) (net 1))
 (segment (start 141.899999 97.200001) (end 135.075001 97.200001) (width 0.25) (layer F.Cu) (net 1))
 (segment (start 135.075001 97.200001) (end 134.25 96.375) (width 0.25) (layer F.Cu) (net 1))
 (segment (start 148 89) (end 147.125 89) (width 0.25) (layer F.Cu) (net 1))
 (segment (start 147.125 89) (end 144 92.125) (width 0.25) (layer F.Cu) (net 1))
 (segment (start 144 92.125) (end 144 92.875) (width 0.25) (layer F.Cu) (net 1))
 (segment (start 144 92.875) (end 144 93.75) (width 0.25) (layer F.Cu) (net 1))
 (segment (start 120.25 62) (end 120.25 61.25) (width 0.25) (layer F.Cu) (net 1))
 (segment (start 120.25 61.25) (end 120.65 60.85) (width 0.25) (layer F.Cu) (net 1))
 (segment (start 120.65 60.85) (end 121.55 60.85) (width 0.25) (layer F.Cu) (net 1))
 (segment (start 121.55 60.85) (end 122.55 60.85) (width 0.25) (layer F.Cu) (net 1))
 (segment (start 142.55 95.85) (end 142.55 95.15) (width 0.25) (layer F.Cu) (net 1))
 (segment (start 142.55 95.15) (end 143.95 93.75) (width 0.25) (layer F.Cu) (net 1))
 (segment (start 143.95 93.75) (end 144 93.75) (width 0.25) (layer F.Cu) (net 1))
 (segment (start 134.25 96.25) (end 134.25 96.375) (width 0.25) (layer F.Cu) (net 1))
 (segment (start 134.25 96.375) (end 132.55 98.075) (width 0.25) (layer F.Cu) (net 1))
 (segment (start 132.55 98.075) (end 132.55 98.35) (width 0.25) (layer F.Cu) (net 1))
 (segment (start 124.25 93.75) (end 124.25 94.45) (width 0.25) (layer F.Cu) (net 1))
 (segment (start 124.25 94.45) (end 122.85 95.85) (width 0.25) (layer F.Cu) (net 1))
 (segment (start 122.85 95.85) (end 122.55 95.85) (width 0.25) (layer F.Cu) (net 1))
 (segment (start 115.05 88.35) (end 115.05 86.7) (width 0.25) (layer F.Cu) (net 1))
 (segment (start 115.05 86.7) (end 115.5 86.25) (width 0.25) (layer F.Cu) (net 1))
 (segment (start 112.55 78.35) (end 112.55 76.95) (width 0.25) (layer F.Cu) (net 1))
 (segment (start 112.55 76.95) (end 113.25 76.25) (width 0.25) (layer F.Cu) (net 1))
 (segment (start 115.05 68.35) (end 115.05 67.65) (width 0.25) (layer F.Cu) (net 1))
 (segment (start 115.05 67.65) (end 116.45 66.25) (width 0.25) (layer F.Cu) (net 1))
 (segment (start 116.45 66.25) (end 116.5 66.25) (width 0.25) (layer F.Cu) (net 1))
 (segment (start 116.5 66.25) (end 117.25 66.25) (width 0.25) (layer F.Cu) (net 1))
 (segment (start 150.05 88.35) (end 148.65 88.35) (width 0.25) (layer F.Cu) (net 1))
 (segment (start 148.65 88.35) (end 148 89) (width 0.25) (layer F.Cu) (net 1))
 (segment (start 152.55 78.35) (end 151.15 78.35) (width 0.25) (layer F.Cu) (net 1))
 (segment (start 151.15 78.35) (end 150.5 79) (width 0.25) (layer F.Cu) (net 1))
 (segment (start 147.75 66.25) (end 149.5 66.25) (width 0.25) (layer F.Cu) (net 1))
 (segment (start 149.5 66.25) (end 150.05 66.8) (width 0.25) (layer F.Cu) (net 1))
 (segment (start 150.05 66.8) (end 150.05 68.35) (width 0.25) (layer F.Cu) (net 1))
 (segment (start 140 60) (end 141.4 60) (width 0.25) (layer F.Cu) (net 1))
 (segment (start 141.4 60) (end 142.25 60.85) (width 0.25) (layer F.Cu) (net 1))
 (segment (start 142.25 60.85) (end 142.55 60.85) (width 0.25) (layer F.Cu) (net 1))
 (segment (start 130.25 59.5) (end 132.1 59.5) (width 0.25) (layer F.Cu) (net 1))
 (segment (start 132.1 59.5) (end 132.55 59.05) (width 0.25) (layer F.Cu) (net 1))
 (segment (start 132.55 59.05) (end 132.55 58.35) (width 0.25) (layer F.Cu) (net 1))
 (segment (start 134.96 82.25) (end 133 82.25) (width 0.25) (layer B.Cu) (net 6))
 (segment (start 136 79.25) (end 136 81.21) (width 0.25) (layer F.Cu) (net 6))
 (segment (start 136 81.21) (end 134.96 82.25) (width 0.25) (layer F.Cu) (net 6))
 (segment (start 141 82.25) (end 140.125 82.25) (width 0.25) (layer B.Cu) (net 7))
 (segment (start 140.125 82.25) (end 137.5 82.25) (width 0.25) (layer B.Cu) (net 7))
 (segment (start 136.8 79.25) (end 136.8 81.55) (width 0.25) (layer F.Cu) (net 7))
 (segment (start 136.8 81.55) (end 137.5 82.25) (width 0.25) (layer F.Cu) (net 7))
 (segment (start 127.45 60.85) (end 127.75 60.85) (width 0.25) (layer F.Cu) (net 28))
 (segment (start 127.75 60.85) (end 132 65.1) (width 0.25) (layer F.Cu) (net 28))
 (segment (start 132 65.1) (end 132 69.7) (width 0.25) (layer F.Cu) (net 28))
 (segment (start 132 69.7) (end 132 70.75) (width 0.25) (layer F.Cu) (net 28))
 (segment (start 129 57) (end 135.1 57) (width 0.25) (layer F.Cu) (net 34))
 (segment (start 135.1 57) (end 136.45 58.35) (width 0.25) (layer F.Cu) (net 34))
 (segment (start 136.45 58.35) (end 137.45 58.35) (width 0.25) (layer F.Cu) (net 34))
 (segment (start 122.55 64.15) (end 122.55 63.45) (width 0.25) (layer F.Cu) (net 34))
 (segment (start 122.55 63.45) (end 129 57) (width 0.25) (layer F.Cu) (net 34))
 (segment (start 132.55 61.65) (end 133.55 61.65) (width 0.25) (layer F.Cu) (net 35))
 (segment (start 133.55 61.65) (end 136.025001 59.174999) (width 0.25) (layer F.Cu) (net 35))
 (segment (start 144.774999 59.174999) (end 146.45 60.85) (width 0.25) (layer F.Cu) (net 35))
 (segment (start 136.025001 59.174999) (end 144.774999 59.174999) (width 0.25) (layer F.Cu) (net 35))
 (segment (start 146.45 60.85) (end 147.45 60.85) (width 0.25) (layer F.Cu) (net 35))
 (segment (start 150.05 91.65) (end 150.05 93.55) (width 0.25) (layer F.Cu) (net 39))
 (segment (start 150.05 93.55) (end 147.75 95.85) (width 0.25) (layer F.Cu) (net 39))
 (segment (start 147.75 95.85) (end 147.45 95.85) (width 0.25) (layer F.Cu) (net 39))
 (segment (start 142.55 64.15) (end 143.55 64.15) (width 0.25) (layer F.Cu) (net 36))
 (segment (start 143.55 64.15) (end 144.7 63) (width 0.25) (layer F.Cu) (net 36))
 (segment (start 144.7 63) (end 150.3 63) (width 0.25) (layer F.Cu) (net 36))
 (segment (start 150.3 63) (end 154.95 67.65) (width 0.25) (layer F.Cu) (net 36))
 (segment (start 154.95 67.65) (end 154.95 68.35) (width 0.25) (layer F.Cu) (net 36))
 (segment (start 152.45 70.25) (end 155.335002 70.25) (width 0.25) (layer F.Cu) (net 37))
 (segment (start 155.335002 70.25) (end 157.45 72.364998) (width 0.25) (layer F.Cu) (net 37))
 (segment (start 157.45 72.364998) (end 157.45 77.65) (width 0.25) (layer F.Cu) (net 37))
 (segment (start 157.45 77.65) (end 157.45 78.35) (width 0.25) (layer F.Cu) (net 37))
 (segment (start 150.05 71.65) (end 151.05 71.65) (width 0.25) (layer F.Cu) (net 37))
 (segment (start 151.05 71.65) (end 152.45 70.25) (width 0.25) (layer F.Cu) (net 37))
 (segment (start 152.55 81.65) (end 153.55 81.65) (width 0.25) (layer F.Cu) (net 38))
 (segment (start 153.55 81.65) (end 154.95 80.25) (width 0.25) (layer F.Cu) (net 38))
 (segment (start 154.95 80.25) (end 157.835002 80.25) (width 0.25) (layer F.Cu) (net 38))
 (segment (start 159.25 81.664998) (end 159.25 84.35) (width 0.25) (layer F.Cu) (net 38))
 (segment (start 157.835002 80.25) (end 159.25 81.664998) (width 0.25) (layer F.Cu) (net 38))
 (segment (start 159.25 84.35) (end 155.25 88.35) (width 0.25) (layer F.Cu) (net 38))
 (segment (start 155.25 88.35) (end 154.95 88.35) (width 0.25) (layer F.Cu) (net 38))
 (segment (start 130.25 97.25) (end 128.85 95.85) (width 0.25) (layer F.Cu) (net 41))
 (segment (start 128.85 95.85) (end 127.45 95.85) (width 0.25) (layer F.Cu) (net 41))
 (segment (start 130.25 100.35) (end 130.25 97.25) (width 0.25) (layer F.Cu) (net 41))
 (segment (start 132.55 101.65) (end 131.55 101.65) (width 0.25) (layer F.Cu) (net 41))
 (segment (start 131.55 101.65) (end 130.25 100.35) (width 0.25) (layer F.Cu) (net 41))
 (segment (start 122.55 99.15) (end 121.55 99.15) (width 0.25) (layer F.Cu) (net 42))
 (segment (start 121.55 99.15) (end 121 98.6) (width 0.25) (layer F.Cu) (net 42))
 (segment (start 122 92) (end 122 90.1) (width 0.25) (layer F.Cu) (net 42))
 (segment (start 121 98.6) (end 121 93) (width 0.25) (layer F.Cu) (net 42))
 (segment (start 121 93) (end 122 92) (width 0.25) (layer F.Cu) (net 42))
 (segment (start 122 90.1) (end 120.25 88.35) (width 0.25) (layer F.Cu) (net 42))
 (segment (start 120.25 88.35) (end 119.95 88.35) (width 0.25) (layer F.Cu) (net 42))
 (segment (start 115.5 82.5) (end 115.5 81) (width 0.25) (layer F.Cu) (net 43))
 (segment (start 115.5 81) (end 117.45 79.05) (width 0.25) (layer F.Cu) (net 43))
 (segment (start 117.45 79.05) (end 117.45 78.35) (width 0.25) (layer F.Cu) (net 43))
 (segment (start 113.85 84.15) (end 115.5 82.5) (width 0.25) (layer F.Cu) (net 43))
 (segment (start 113.85 89.75) (end 113.85 84.15) (width 0.25) (layer F.Cu) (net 43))
 (segment (start 115.05 91.65) (end 115.05 90.95) (width 0.25) (layer F.Cu) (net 43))
 (segment (start 115.05 90.95) (end 113.85 89.75) (width 0.25) (layer F.Cu) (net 43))
 (segment (start 140.9 99.15) (end 140.1 98.35) (width 0.25) (layer F.Cu) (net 40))
 (segment (start 140.1 98.35) (end 137.45 98.35) (width 0.25) (layer F.Cu) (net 40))
 (segment (start 142.55 99.15) (end 140.9 99.15) (width 0.25) (layer F.Cu) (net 40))
 (segment (start 115.75 73.25) (end 119.95 69.05) (width 0.25) (layer F.Cu) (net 44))
 (segment (start 119.95 69.05) (end 119.95 68.35) (width 0.25) (layer F.Cu) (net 44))
 (segment (start 114 73.25) (end 115.75 73.25) (width 0.25) (layer F.Cu) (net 44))
 (segment (start 111 76.25) (end 114 73.25) (width 0.25) (layer F.Cu) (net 44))
 (segment (start 111 79.4) (end 111 76.25) (width 0.25) (layer F.Cu) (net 44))
 (segment (start 112.55 81.65) (end 112.55 80.95) (width 0.25) (layer F.Cu) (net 44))
 (segment (start 112.55 80.95) (end 111 79.4) (width 0.25) (layer F.Cu) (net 44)))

